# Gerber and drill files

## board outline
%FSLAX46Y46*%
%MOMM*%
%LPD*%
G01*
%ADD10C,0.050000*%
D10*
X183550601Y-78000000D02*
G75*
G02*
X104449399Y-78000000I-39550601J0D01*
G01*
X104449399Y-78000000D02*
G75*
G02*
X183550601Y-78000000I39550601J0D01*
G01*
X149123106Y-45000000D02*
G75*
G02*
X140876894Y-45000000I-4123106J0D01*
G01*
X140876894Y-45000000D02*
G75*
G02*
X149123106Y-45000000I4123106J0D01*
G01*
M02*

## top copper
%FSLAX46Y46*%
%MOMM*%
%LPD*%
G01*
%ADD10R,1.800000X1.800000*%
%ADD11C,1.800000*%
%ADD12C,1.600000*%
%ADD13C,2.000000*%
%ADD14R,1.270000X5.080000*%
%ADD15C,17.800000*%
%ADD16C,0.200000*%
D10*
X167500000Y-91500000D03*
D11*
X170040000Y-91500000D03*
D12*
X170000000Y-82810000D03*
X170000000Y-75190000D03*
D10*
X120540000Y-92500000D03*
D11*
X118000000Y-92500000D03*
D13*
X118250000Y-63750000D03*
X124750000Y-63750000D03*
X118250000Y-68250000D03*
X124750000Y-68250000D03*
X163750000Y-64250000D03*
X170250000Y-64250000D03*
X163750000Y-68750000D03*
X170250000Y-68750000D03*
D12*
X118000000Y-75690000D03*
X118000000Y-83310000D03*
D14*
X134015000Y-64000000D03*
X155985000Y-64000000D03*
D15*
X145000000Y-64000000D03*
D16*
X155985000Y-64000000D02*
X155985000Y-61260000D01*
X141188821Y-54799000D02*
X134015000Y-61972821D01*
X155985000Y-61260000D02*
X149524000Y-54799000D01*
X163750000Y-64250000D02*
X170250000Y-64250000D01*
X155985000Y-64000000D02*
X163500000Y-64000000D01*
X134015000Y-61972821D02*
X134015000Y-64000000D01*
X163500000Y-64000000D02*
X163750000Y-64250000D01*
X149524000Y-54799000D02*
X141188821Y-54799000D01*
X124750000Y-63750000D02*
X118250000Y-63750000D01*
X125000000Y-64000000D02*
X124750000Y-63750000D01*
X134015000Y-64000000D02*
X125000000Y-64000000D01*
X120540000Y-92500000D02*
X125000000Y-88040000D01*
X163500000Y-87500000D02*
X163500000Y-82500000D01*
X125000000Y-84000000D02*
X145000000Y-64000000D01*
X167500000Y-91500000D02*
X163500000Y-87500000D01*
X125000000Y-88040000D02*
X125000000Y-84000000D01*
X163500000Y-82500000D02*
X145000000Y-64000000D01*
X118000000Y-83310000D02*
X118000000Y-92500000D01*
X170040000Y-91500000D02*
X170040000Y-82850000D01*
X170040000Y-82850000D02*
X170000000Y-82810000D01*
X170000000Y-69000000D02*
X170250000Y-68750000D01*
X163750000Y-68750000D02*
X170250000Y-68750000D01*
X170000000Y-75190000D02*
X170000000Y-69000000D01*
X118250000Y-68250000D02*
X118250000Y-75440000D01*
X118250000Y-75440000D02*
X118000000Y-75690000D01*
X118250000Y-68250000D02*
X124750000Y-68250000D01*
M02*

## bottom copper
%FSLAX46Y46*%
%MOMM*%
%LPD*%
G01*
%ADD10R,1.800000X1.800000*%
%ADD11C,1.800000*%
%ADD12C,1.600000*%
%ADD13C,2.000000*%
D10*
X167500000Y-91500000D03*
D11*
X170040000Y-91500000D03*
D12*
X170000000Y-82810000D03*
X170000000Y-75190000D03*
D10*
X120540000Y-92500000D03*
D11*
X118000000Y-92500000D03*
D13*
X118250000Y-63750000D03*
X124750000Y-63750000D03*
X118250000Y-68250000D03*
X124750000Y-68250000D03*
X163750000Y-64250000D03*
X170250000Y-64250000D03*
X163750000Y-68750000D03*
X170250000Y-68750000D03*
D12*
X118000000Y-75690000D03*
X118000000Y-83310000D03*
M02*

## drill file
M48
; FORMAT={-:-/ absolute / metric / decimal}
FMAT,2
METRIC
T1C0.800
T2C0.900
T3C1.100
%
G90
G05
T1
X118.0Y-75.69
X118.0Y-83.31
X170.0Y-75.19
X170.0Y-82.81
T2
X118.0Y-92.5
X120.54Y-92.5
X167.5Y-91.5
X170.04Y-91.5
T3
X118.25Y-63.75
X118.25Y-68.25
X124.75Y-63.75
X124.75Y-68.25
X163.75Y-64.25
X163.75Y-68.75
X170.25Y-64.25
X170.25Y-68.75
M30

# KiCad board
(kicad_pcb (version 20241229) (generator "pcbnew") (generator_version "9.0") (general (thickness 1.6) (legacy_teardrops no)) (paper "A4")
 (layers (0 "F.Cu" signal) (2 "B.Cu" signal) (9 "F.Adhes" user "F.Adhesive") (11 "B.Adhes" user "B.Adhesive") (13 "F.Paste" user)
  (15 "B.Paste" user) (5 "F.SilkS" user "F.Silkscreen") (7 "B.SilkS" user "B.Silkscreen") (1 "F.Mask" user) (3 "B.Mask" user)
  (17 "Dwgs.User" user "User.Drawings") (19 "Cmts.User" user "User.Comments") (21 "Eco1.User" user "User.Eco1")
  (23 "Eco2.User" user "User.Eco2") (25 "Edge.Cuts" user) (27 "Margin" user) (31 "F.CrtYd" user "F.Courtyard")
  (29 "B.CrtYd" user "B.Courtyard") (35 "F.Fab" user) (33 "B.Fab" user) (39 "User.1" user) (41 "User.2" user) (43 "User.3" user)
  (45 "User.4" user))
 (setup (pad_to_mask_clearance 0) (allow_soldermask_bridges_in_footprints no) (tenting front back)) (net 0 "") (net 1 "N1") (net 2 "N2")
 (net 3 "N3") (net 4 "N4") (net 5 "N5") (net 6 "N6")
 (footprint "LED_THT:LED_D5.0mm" (layer "F.Cu") (at 167.5 91.5)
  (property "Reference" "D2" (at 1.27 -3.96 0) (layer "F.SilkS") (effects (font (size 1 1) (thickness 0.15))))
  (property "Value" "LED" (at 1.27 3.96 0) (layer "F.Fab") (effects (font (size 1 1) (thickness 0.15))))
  (pad "1" thru_hole rect (at 0 0) (size 1.8 1.8) (drill 0.9) (layers "*.Cu" "*.Mask") (remove_unused_layers no) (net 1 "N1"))
  (pad "2" thru_hole circle (at 2.54 0) (size 1.8 1.8) (drill 0.9) (layers "*.Cu" "*.Mask") (remove_unused_layers no) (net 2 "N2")))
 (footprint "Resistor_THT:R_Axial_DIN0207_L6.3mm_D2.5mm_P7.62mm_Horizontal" (layer "F.Cu") (at 170 82.81 90)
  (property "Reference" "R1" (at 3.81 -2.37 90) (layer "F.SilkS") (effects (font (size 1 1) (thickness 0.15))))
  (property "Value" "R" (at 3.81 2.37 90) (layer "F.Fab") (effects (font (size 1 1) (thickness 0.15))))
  (pad "1" thru_hole circle (at 0 0 90) (size 1.6 1.6) (drill 0.8) (layers "*.Cu" "*.Mask") (remove_unused_layers no) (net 2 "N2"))
  (pad "2" thru_hole circle (at 7.62 0 90) (size 1.6 1.6) (drill 0.8) (layers "*.Cu" "*.Mask") (remove_unused_layers no) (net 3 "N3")))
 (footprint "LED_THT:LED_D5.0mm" (layer "F.Cu") (at 120.54 92.5 180)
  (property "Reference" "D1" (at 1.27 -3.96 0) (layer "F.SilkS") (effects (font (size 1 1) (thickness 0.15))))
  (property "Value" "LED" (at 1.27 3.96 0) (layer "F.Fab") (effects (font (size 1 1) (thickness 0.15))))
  (pad "1" thru_hole rect (at 0 0 180) (size 1.8 1.8) (drill 0.9) (layers "*.Cu" "*.Mask") (remove_unused_layers no) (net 1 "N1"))
  (pad "2" thru_hole circle (at 2.54 0 180) (size 1.8 1.8) (drill 0.9) (layers "*.Cu" "*.Mask") (remove_unused_layers no) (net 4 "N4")))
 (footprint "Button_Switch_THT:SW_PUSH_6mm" (layer "F.Cu") (at 118.25 63.75)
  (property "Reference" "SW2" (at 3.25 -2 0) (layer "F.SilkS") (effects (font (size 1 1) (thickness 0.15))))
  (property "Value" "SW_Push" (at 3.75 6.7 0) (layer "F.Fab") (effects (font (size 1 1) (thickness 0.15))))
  (pad "1" thru_hole circle (at 0 0 90) (size 2 2) (drill 1.1) (layers "*.Cu" "*.Mask") (remove_unused_layers no) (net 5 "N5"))
  (pad "1" thru_hole circle (at 6.5 0 90) (size 2 2) (drill 1.1) (layers "*.Cu" "*.Mask") (remove_unused_layers no) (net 5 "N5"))
  (pad "2" thru_hole circle (at 0 4.5 90) (size 2 2) (drill 1.1) (layers "*.Cu" "*.Mask") (remove_unused_layers no) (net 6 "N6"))
  (pad "2" thru_hole circle (at 6.5 4.5 90) (size 2 2) (drill 1.1) (layers "*.Cu" "*.Mask") (remove_unused_layers no) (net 6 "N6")))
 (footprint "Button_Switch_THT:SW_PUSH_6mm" (layer "F.Cu") (at 163.75 64.25)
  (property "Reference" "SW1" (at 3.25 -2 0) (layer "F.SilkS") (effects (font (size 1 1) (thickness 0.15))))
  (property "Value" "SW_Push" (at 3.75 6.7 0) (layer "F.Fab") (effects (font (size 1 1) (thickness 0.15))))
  (pad "1" thru_hole circle (at 0 0 90) (size 2 2) (drill 1.1) (layers "*.Cu" "*.Mask") (remove_unused_layers no) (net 5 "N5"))
  (pad "1" thru_hole circle (at 6.5 0 90) (size 2 2) (drill 1.1) (layers "*.Cu" "*.Mask") (remove_unused_layers no) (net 5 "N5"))
  (pad "2" thru_hole circle (at 0 4.5 90) (size 2 2) (drill 1.1) (layers "*.Cu" "*.Mask") (remove_unused_layers no) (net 3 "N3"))
  (pad "2" thru_hole circle (at 6.5 4.5 90) (size 2 2) (drill 1.1) (layers "*.Cu" "*.Mask") (remove_unused_layers no) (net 3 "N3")))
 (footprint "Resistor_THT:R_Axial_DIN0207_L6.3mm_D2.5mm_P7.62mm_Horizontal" (layer "F.Cu") (at 118 75.69 -90)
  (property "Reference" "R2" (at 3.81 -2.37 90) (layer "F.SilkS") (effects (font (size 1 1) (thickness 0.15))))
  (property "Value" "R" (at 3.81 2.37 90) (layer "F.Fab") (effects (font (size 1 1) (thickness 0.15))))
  (pad "1" thru_hole circle (at 0 0 270) (size 1.6 1.6) (drill 0.8) (layers "*.Cu" "*.Mask") (remove_unused_layers no) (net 6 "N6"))
  (pad "2" thru_hole circle (at 7.62 0 270) (size 1.6 1.6) (drill 0.8) (layers "*.Cu" "*.Mask") (remove_unused_layers no) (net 4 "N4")))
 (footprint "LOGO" (layer "F.Cu") (at 145.5 94)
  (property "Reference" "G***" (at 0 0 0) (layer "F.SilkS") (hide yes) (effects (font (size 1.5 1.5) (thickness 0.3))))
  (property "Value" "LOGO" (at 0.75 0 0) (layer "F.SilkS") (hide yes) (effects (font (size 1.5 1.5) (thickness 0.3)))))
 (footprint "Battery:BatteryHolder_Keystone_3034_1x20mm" (layer "F.Cu") (at 145 64)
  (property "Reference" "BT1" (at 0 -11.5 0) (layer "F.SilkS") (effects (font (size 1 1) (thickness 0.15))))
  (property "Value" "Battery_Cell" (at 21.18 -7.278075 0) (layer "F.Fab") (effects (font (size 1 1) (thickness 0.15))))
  (pad "1" smd rect (at -10.985 0) (size 1.27 5.08) (layers "F.Cu" "F.Mask" "F.Paste") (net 5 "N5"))
  (pad "1" smd rect (at 10.985 0) (size 1.27 5.08) (layers "F.Cu" "F.Mask" "F.Paste") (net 5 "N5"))
  (pad "2" smd circle (at 0 0) (size 17.8 17.8) (layers "F.Cu" "F.Mask") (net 1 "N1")))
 (gr_circle (center 144 78) (end 183.5 76) (stroke (width 0.05) (type default)) (fill no) (layer "Edge.Cuts"))
 (gr_circle (center 145 45) (end 149 46) (stroke (width 0.05) (type default)) (fill no) (layer "Edge.Cuts"))
 (segment (start 155.985 64) (end 155.985 61.26) (width 0.2) (layer "F.Cu") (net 5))
 (segment (start 141.188821 54.799) (end 134.015 61.972821) (width 0.2) (layer "F.Cu") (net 5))
 (segment (start 155.985 61.26) (end 149.524 54.799) (width 0.2) (layer "F.Cu") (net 5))
 (segment (start 163.75 64.25) (end 170.25 64.25) (width 0.2) (layer "F.Cu") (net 5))
 (segment (start 155.985 64) (end 163.5 64) (width 0.2) (layer "F.Cu") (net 5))
 (segment (start 134.015 61.972821) (end 134.015 64) (width 0.2) (layer "F.Cu") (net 5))
 (segment (start 163.5 64) (end 163.75 64.25) (width 0.2) (layer "F.Cu") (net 5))
 (segment (start 149.524 54.799) (end 141.188821 54.799) (width 0.2) (layer "F.Cu") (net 5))
 (segment (start 124.75 63.75) (end 118.25 63.75) (width 0.2) (layer "F.Cu") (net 5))
 (segment (start 125 64) (end 124.75 63.75) (width 0.2) (layer "F.Cu") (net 5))
 (segment (start 134.015 64) (end 125 64) (width 0.2) (layer "F.Cu") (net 5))
 (segment (start 120.54 92.5) (end 125 88.04) (width 0.2) (layer "F.Cu") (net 1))
 (segment (start 163.5 87.5) (end 163.5 82.5) (width 0.2) (layer "F.Cu") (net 1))
 (segment (start 125 84) (end 145 64) (width 0.2) (layer "F.Cu") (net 1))
 (segment (start 167.5 91.5) (end 163.5 87.5) (width 0.2) (layer "F.Cu") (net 1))
 (segment (start 125 88.04) (end 125 84) (width 0.2) (layer "F.Cu") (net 1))
 (segment (start 163.5 82.5) (end 145 64) (width 0.2) (layer "F.Cu") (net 1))
 (segment (start 118 83.31) (end 118 92.5) (width 0.2) (layer "F.Cu") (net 4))
 (segment (start 170.04 91.5) (end 170.04 82.85) (width 0.2) (layer "F.Cu") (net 2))
 (segment (start 170.04 82.85) (end 170 82.81) (width 0.2) (layer "F.Cu") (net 2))
 (segment (start 170 69) (end 170.25 68.75) (width 0.2) (layer "F.Cu") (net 3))
 (segment (start 163.75 68.75) (end 170.25 68.75) (width 0.2) (layer "F.Cu") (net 3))
 (segment (start 170 75.19) (end 170 69) (width 0.2) (layer "F.Cu") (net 3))
 (segment (start 118.25 68.25) (end 118.25 75.44) (width 0.2) (layer "F.Cu") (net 6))
 (segment (start 118.25 75.44) (end 118 75.69) (width 0.2) (layer "F.Cu") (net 6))
 (segment (start 118.25 68.25) (end 124.75 68.25) (width 0.2) (layer "F.Cu") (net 6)))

